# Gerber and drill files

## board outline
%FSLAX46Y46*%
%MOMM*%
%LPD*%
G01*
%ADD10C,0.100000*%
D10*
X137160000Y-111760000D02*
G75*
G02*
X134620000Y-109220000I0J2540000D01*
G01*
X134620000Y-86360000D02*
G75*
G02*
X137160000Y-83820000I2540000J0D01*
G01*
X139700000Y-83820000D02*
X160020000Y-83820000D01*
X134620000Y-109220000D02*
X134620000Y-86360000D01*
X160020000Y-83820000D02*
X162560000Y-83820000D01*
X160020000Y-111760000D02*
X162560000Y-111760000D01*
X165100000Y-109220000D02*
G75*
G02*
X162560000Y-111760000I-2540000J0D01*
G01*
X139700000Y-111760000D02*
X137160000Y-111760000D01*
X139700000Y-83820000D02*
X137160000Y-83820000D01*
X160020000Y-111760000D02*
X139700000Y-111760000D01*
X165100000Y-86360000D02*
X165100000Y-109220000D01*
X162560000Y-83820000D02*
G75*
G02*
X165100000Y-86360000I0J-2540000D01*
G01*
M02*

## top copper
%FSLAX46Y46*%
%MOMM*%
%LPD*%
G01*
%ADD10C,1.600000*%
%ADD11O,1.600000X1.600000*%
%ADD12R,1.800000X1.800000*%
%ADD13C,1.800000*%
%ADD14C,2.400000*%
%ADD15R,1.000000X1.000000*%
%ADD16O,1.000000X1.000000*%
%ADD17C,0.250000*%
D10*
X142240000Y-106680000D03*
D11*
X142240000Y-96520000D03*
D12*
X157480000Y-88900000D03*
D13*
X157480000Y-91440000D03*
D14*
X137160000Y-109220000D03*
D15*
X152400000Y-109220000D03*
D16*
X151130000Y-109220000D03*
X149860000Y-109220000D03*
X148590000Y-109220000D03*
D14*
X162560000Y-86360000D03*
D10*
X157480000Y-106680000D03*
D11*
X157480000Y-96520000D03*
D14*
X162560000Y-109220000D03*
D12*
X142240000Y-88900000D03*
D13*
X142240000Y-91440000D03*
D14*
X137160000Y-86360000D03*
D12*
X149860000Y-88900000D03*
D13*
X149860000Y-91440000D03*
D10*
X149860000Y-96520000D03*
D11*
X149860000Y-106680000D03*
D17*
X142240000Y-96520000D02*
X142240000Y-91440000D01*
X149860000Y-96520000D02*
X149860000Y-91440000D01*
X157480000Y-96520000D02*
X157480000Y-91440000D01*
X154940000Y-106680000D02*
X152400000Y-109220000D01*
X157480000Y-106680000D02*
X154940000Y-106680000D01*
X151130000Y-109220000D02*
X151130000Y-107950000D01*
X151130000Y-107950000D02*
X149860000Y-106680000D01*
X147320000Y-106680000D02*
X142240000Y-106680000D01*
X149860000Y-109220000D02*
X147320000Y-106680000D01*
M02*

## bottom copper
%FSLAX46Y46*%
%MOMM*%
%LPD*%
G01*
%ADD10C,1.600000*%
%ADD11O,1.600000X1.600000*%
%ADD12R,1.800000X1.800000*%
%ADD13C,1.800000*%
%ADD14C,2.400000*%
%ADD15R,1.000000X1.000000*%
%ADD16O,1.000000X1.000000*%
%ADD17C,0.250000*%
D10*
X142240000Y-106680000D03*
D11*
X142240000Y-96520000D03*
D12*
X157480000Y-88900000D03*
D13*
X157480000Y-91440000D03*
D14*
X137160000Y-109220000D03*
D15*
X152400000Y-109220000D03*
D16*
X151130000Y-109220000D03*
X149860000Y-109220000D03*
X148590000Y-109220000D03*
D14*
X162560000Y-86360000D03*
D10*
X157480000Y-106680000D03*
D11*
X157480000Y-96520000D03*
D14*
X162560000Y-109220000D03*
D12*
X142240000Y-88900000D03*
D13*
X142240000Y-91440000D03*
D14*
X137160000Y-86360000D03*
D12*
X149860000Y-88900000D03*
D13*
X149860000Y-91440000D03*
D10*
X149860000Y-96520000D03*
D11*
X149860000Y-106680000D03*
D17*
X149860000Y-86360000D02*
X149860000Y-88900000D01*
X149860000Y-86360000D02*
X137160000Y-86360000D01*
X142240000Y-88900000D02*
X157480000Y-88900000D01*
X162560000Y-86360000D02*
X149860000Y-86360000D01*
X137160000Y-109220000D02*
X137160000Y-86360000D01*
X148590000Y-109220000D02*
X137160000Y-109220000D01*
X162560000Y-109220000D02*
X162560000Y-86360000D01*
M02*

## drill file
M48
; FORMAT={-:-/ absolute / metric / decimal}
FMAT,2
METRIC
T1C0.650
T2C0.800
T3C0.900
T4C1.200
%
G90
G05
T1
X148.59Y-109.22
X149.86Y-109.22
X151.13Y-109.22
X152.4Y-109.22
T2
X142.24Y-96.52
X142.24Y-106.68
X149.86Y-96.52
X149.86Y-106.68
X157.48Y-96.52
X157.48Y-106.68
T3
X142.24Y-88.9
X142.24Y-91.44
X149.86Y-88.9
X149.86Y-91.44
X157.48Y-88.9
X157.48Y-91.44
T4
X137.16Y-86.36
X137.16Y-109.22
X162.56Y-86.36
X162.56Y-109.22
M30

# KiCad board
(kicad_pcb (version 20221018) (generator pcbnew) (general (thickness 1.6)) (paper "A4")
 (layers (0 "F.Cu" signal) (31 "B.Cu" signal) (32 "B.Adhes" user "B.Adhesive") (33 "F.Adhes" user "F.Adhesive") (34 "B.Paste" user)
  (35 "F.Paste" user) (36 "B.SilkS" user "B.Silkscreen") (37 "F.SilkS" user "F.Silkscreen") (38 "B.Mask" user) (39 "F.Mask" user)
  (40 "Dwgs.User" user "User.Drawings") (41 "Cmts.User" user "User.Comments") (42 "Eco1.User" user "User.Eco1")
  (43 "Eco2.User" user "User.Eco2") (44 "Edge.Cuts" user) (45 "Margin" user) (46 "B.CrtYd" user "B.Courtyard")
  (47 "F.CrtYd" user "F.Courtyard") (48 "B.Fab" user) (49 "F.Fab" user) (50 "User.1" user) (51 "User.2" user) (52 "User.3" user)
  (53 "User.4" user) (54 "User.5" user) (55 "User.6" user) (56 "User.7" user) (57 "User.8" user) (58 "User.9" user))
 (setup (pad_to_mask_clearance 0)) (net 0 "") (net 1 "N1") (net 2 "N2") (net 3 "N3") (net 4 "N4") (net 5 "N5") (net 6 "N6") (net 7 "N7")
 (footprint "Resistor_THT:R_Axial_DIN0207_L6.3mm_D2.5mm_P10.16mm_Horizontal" (layer "F.Cu") (at 142.24 106.68 90)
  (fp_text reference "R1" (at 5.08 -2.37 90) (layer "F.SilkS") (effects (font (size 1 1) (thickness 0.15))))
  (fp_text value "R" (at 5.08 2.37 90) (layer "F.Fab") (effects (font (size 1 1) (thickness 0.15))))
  (pad "1" thru_hole circle (at 0 0 90) (size 1.6 1.6) (drill 0.8) (layers "*.Cu" "*.Mask") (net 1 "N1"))
  (pad "2" thru_hole oval (at 10.16 0 90) (size 1.6 1.6) (drill 0.8) (layers "*.Cu" "*.Mask") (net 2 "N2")))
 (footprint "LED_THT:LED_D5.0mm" (layer "F.Cu") (at 157.48 88.9 -90)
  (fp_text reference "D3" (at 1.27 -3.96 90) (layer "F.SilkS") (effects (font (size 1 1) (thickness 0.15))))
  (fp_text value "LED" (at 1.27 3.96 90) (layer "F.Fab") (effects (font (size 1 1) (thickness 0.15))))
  (pad "1" thru_hole rect (at 0 0 270) (size 1.8 1.8) (drill 0.9) (layers "*.Cu" "*.Mask") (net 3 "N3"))
  (pad "2" thru_hole circle (at 2.54 0 270) (size 1.8 1.8) (drill 0.9) (layers "*.Cu" "*.Mask") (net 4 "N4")))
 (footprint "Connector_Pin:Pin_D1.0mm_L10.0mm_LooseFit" (layer "F.Cu") (at 137.16 109.22)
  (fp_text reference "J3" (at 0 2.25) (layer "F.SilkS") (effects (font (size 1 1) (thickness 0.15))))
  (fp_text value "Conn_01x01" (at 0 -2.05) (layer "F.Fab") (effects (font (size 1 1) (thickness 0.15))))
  (pad "1" thru_hole circle (at 0 0) (size 2.4 2.4) (drill 1.2) (layers "*.Cu" "*.Mask") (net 3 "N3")))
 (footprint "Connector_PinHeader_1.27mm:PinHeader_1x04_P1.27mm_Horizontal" (layer "F.Cu") (at 152.4 109.22 -90)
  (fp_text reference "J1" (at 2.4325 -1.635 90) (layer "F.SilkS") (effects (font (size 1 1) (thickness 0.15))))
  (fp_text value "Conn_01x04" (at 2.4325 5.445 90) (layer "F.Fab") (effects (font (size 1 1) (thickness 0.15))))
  (pad "1" thru_hole rect (at 0 0 270) (size 1 1) (drill 0.65) (layers "*.Cu" "*.Mask") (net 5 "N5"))
  (pad "2" thru_hole oval (at 0 1.27 270) (size 1 1) (drill 0.65) (layers "*.Cu" "*.Mask") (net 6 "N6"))
  (pad "3" thru_hole oval (at 0 2.54 270) (size 1 1) (drill 0.65) (layers "*.Cu" "*.Mask") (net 1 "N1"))
  (pad "4" thru_hole oval (at 0 3.81 270) (size 1 1) (drill 0.65) (layers "*.Cu" "*.Mask") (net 3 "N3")))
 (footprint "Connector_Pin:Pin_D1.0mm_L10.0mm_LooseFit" (layer "F.Cu") (at 162.56 86.36)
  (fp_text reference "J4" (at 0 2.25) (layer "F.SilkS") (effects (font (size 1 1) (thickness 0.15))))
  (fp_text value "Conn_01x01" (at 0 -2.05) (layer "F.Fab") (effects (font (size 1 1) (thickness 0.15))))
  (pad "1" thru_hole circle (at 0 0) (size 2.4 2.4) (drill 1.2) (layers "*.Cu" "*.Mask") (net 3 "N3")))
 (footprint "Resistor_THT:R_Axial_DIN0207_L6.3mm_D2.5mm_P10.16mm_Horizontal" (layer "F.Cu") (at 157.48 106.68 90)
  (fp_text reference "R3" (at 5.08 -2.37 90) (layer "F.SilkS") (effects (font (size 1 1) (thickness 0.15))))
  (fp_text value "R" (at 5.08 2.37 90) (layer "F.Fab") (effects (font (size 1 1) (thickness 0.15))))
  (pad "1" thru_hole circle (at 0 0 90) (size 1.6 1.6) (drill 0.8) (layers "*.Cu" "*.Mask") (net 5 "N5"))
  (pad "2" thru_hole oval (at 10.16 0 90) (size 1.6 1.6) (drill 0.8) (layers "*.Cu" "*.Mask") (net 4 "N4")))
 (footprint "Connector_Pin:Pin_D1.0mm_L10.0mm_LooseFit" (layer "F.Cu") (at 162.56 109.22)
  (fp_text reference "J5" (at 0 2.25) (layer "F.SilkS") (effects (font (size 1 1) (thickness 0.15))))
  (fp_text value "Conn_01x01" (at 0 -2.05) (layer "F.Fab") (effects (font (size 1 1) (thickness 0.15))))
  (pad "1" thru_hole circle (at 0 0) (size 2.4 2.4) (drill 1.2) (layers "*.Cu" "*.Mask") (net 3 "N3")))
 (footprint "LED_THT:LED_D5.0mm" (layer "F.Cu") (at 142.24 88.9 -90)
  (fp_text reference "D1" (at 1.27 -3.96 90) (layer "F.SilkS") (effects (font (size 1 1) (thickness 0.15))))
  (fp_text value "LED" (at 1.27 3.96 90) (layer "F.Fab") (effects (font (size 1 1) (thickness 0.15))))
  (pad "1" thru_hole rect (at 0 0 270) (size 1.8 1.8) (drill 0.9) (layers "*.Cu" "*.Mask") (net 3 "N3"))
  (pad "2" thru_hole circle (at 2.54 0 270) (size 1.8 1.8) (drill 0.9) (layers "*.Cu" "*.Mask") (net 2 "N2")))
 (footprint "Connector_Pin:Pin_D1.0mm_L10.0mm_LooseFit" (layer "F.Cu") (at 137.16 86.36)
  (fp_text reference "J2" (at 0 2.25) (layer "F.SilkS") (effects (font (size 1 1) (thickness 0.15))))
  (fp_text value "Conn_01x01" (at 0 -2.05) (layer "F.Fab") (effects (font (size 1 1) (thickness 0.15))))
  (pad "1" thru_hole circle (at 0 0) (size 2.4 2.4) (drill 1.2) (layers "*.Cu" "*.Mask") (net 3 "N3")))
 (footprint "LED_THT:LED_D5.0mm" (layer "F.Cu") (at 149.86 88.9 -90)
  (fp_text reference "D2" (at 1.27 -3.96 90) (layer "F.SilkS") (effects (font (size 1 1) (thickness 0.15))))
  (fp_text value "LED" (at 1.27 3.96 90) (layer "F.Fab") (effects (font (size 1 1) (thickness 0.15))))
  (pad "1" thru_hole rect (at 0 0 270) (size 1.8 1.8) (drill 0.9) (layers "*.Cu" "*.Mask") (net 3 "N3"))
  (pad "2" thru_hole circle (at 2.54 0 270) (size 1.8 1.8) (drill 0.9) (layers "*.Cu" "*.Mask") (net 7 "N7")))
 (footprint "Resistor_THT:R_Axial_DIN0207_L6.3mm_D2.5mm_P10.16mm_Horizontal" (layer "F.Cu") (at 149.86 96.52 -90)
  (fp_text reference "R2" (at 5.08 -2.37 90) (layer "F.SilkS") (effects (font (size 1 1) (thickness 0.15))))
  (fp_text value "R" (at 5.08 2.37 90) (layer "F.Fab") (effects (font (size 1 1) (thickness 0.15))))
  (pad "1" thru_hole circle (at 0 0 270) (size 1.6 1.6) (drill 0.8) (layers "*.Cu" "*.Mask") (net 7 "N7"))
  (pad "2" thru_hole oval (at 10.16 0 270) (size 1.6 1.6) (drill 0.8) (layers "*.Cu" "*.Mask") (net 6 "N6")))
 (gr_arc (start 137.16 111.76) (mid 135.363949 111.016051) (end 134.62 109.22) (stroke (width 0.1) (type default)) (layer "Edge.Cuts"))
 (gr_arc (start 134.62 86.36) (mid 135.363949 84.563949) (end 137.16 83.82) (stroke (width 0.1) (type default)) (layer "Edge.Cuts"))
 (gr_line (start 139.7 83.82) (end 160.02 83.82) (stroke (width 0.1) (type default)) (layer "Edge.Cuts"))
 (gr_line (start 134.62 109.22) (end 134.62 86.36) (stroke (width 0.1) (type default)) (layer "Edge.Cuts"))
 (gr_line (start 160.02 83.82) (end 162.56 83.82) (stroke (width 0.1) (type default)) (layer "Edge.Cuts"))
 (gr_line (start 160.02 111.76) (end 162.56 111.76) (stroke (width 0.1) (type default)) (layer "Edge.Cuts"))
 (gr_arc (start 165.1 109.22) (mid 164.356051 111.016051) (end 162.56 111.76) (stroke (width 0.1) (type default)) (layer "Edge.Cuts"))
 (gr_line (start 139.7 111.76) (end 137.16 111.76) (stroke (width 0.1) (type default)) (layer "Edge.Cuts"))
 (gr_line (start 139.7 83.82) (end 137.16 83.82) (stroke (width 0.1) (type default)) (layer "Edge.Cuts"))
 (gr_line (start 160.02 111.76) (end 139.7 111.76) (stroke (width 0.1) (type default)) (layer "Edge.Cuts"))
 (gr_line (start 165.1 86.36) (end 165.1 109.22) (stroke (width 0.1) (type default)) (layer "Edge.Cuts"))
 (gr_arc (start 162.56 83.82) (mid 164.356051 84.563949) (end 165.1 86.36) (stroke (width 0.1) (type default)) (layer "Edge.Cuts"))
 (segment (start 149.86 86.36) (end 149.86 88.9) (width 0.25) (layer "B.Cu") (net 3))
 (segment (start 149.86 86.36) (end 137.16 86.36) (width 0.25) (layer "B.Cu") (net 3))
 (segment (start 142.24 88.9) (end 157.48 88.9) (width 0.25) (layer "B.Cu") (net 3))
 (segment (start 162.56 86.36) (end 149.86 86.36) (width 0.25) (layer "B.Cu") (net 3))
 (segment (start 137.16 109.22) (end 137.16 86.36) (width 0.25) (layer "B.Cu") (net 3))
 (segment (start 148.59 109.22) (end 137.16 109.22) (width 0.25) (layer "B.Cu") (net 3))
 (segment (start 162.56 109.22) (end 162.56 86.36) (width 0.25) (layer "B.Cu") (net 3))
 (segment (start 142.24 96.52) (end 142.24 91.44) (width 0.25) (layer "F.Cu") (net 2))
 (segment (start 149.86 96.52) (end 149.86 91.44) (width 0.25) (layer "F.Cu") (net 7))
 (segment (start 157.48 96.52) (end 157.48 91.44) (width 0.25) (layer "F.Cu") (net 4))
 (segment (start 154.94 106.68) (end 152.4 109.22) (width 0.25) (layer "F.Cu") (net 5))
 (segment (start 157.48 106.68) (end 154.94 106.68) (width 0.25) (layer "F.Cu") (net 5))
 (segment (start 151.13 109.22) (end 151.13 107.95) (width 0.25) (layer "F.Cu") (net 6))
 (segment (start 151.13 107.95) (end 149.86 106.68) (width 0.25) (layer "F.Cu") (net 6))
 (segment (start 147.32 106.68) (end 142.24 106.68) (width 0.25) (layer "F.Cu") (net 1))
 (segment (start 149.86 109.22) (end 147.32 106.68) (width 0.25) (layer "F.Cu") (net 1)))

